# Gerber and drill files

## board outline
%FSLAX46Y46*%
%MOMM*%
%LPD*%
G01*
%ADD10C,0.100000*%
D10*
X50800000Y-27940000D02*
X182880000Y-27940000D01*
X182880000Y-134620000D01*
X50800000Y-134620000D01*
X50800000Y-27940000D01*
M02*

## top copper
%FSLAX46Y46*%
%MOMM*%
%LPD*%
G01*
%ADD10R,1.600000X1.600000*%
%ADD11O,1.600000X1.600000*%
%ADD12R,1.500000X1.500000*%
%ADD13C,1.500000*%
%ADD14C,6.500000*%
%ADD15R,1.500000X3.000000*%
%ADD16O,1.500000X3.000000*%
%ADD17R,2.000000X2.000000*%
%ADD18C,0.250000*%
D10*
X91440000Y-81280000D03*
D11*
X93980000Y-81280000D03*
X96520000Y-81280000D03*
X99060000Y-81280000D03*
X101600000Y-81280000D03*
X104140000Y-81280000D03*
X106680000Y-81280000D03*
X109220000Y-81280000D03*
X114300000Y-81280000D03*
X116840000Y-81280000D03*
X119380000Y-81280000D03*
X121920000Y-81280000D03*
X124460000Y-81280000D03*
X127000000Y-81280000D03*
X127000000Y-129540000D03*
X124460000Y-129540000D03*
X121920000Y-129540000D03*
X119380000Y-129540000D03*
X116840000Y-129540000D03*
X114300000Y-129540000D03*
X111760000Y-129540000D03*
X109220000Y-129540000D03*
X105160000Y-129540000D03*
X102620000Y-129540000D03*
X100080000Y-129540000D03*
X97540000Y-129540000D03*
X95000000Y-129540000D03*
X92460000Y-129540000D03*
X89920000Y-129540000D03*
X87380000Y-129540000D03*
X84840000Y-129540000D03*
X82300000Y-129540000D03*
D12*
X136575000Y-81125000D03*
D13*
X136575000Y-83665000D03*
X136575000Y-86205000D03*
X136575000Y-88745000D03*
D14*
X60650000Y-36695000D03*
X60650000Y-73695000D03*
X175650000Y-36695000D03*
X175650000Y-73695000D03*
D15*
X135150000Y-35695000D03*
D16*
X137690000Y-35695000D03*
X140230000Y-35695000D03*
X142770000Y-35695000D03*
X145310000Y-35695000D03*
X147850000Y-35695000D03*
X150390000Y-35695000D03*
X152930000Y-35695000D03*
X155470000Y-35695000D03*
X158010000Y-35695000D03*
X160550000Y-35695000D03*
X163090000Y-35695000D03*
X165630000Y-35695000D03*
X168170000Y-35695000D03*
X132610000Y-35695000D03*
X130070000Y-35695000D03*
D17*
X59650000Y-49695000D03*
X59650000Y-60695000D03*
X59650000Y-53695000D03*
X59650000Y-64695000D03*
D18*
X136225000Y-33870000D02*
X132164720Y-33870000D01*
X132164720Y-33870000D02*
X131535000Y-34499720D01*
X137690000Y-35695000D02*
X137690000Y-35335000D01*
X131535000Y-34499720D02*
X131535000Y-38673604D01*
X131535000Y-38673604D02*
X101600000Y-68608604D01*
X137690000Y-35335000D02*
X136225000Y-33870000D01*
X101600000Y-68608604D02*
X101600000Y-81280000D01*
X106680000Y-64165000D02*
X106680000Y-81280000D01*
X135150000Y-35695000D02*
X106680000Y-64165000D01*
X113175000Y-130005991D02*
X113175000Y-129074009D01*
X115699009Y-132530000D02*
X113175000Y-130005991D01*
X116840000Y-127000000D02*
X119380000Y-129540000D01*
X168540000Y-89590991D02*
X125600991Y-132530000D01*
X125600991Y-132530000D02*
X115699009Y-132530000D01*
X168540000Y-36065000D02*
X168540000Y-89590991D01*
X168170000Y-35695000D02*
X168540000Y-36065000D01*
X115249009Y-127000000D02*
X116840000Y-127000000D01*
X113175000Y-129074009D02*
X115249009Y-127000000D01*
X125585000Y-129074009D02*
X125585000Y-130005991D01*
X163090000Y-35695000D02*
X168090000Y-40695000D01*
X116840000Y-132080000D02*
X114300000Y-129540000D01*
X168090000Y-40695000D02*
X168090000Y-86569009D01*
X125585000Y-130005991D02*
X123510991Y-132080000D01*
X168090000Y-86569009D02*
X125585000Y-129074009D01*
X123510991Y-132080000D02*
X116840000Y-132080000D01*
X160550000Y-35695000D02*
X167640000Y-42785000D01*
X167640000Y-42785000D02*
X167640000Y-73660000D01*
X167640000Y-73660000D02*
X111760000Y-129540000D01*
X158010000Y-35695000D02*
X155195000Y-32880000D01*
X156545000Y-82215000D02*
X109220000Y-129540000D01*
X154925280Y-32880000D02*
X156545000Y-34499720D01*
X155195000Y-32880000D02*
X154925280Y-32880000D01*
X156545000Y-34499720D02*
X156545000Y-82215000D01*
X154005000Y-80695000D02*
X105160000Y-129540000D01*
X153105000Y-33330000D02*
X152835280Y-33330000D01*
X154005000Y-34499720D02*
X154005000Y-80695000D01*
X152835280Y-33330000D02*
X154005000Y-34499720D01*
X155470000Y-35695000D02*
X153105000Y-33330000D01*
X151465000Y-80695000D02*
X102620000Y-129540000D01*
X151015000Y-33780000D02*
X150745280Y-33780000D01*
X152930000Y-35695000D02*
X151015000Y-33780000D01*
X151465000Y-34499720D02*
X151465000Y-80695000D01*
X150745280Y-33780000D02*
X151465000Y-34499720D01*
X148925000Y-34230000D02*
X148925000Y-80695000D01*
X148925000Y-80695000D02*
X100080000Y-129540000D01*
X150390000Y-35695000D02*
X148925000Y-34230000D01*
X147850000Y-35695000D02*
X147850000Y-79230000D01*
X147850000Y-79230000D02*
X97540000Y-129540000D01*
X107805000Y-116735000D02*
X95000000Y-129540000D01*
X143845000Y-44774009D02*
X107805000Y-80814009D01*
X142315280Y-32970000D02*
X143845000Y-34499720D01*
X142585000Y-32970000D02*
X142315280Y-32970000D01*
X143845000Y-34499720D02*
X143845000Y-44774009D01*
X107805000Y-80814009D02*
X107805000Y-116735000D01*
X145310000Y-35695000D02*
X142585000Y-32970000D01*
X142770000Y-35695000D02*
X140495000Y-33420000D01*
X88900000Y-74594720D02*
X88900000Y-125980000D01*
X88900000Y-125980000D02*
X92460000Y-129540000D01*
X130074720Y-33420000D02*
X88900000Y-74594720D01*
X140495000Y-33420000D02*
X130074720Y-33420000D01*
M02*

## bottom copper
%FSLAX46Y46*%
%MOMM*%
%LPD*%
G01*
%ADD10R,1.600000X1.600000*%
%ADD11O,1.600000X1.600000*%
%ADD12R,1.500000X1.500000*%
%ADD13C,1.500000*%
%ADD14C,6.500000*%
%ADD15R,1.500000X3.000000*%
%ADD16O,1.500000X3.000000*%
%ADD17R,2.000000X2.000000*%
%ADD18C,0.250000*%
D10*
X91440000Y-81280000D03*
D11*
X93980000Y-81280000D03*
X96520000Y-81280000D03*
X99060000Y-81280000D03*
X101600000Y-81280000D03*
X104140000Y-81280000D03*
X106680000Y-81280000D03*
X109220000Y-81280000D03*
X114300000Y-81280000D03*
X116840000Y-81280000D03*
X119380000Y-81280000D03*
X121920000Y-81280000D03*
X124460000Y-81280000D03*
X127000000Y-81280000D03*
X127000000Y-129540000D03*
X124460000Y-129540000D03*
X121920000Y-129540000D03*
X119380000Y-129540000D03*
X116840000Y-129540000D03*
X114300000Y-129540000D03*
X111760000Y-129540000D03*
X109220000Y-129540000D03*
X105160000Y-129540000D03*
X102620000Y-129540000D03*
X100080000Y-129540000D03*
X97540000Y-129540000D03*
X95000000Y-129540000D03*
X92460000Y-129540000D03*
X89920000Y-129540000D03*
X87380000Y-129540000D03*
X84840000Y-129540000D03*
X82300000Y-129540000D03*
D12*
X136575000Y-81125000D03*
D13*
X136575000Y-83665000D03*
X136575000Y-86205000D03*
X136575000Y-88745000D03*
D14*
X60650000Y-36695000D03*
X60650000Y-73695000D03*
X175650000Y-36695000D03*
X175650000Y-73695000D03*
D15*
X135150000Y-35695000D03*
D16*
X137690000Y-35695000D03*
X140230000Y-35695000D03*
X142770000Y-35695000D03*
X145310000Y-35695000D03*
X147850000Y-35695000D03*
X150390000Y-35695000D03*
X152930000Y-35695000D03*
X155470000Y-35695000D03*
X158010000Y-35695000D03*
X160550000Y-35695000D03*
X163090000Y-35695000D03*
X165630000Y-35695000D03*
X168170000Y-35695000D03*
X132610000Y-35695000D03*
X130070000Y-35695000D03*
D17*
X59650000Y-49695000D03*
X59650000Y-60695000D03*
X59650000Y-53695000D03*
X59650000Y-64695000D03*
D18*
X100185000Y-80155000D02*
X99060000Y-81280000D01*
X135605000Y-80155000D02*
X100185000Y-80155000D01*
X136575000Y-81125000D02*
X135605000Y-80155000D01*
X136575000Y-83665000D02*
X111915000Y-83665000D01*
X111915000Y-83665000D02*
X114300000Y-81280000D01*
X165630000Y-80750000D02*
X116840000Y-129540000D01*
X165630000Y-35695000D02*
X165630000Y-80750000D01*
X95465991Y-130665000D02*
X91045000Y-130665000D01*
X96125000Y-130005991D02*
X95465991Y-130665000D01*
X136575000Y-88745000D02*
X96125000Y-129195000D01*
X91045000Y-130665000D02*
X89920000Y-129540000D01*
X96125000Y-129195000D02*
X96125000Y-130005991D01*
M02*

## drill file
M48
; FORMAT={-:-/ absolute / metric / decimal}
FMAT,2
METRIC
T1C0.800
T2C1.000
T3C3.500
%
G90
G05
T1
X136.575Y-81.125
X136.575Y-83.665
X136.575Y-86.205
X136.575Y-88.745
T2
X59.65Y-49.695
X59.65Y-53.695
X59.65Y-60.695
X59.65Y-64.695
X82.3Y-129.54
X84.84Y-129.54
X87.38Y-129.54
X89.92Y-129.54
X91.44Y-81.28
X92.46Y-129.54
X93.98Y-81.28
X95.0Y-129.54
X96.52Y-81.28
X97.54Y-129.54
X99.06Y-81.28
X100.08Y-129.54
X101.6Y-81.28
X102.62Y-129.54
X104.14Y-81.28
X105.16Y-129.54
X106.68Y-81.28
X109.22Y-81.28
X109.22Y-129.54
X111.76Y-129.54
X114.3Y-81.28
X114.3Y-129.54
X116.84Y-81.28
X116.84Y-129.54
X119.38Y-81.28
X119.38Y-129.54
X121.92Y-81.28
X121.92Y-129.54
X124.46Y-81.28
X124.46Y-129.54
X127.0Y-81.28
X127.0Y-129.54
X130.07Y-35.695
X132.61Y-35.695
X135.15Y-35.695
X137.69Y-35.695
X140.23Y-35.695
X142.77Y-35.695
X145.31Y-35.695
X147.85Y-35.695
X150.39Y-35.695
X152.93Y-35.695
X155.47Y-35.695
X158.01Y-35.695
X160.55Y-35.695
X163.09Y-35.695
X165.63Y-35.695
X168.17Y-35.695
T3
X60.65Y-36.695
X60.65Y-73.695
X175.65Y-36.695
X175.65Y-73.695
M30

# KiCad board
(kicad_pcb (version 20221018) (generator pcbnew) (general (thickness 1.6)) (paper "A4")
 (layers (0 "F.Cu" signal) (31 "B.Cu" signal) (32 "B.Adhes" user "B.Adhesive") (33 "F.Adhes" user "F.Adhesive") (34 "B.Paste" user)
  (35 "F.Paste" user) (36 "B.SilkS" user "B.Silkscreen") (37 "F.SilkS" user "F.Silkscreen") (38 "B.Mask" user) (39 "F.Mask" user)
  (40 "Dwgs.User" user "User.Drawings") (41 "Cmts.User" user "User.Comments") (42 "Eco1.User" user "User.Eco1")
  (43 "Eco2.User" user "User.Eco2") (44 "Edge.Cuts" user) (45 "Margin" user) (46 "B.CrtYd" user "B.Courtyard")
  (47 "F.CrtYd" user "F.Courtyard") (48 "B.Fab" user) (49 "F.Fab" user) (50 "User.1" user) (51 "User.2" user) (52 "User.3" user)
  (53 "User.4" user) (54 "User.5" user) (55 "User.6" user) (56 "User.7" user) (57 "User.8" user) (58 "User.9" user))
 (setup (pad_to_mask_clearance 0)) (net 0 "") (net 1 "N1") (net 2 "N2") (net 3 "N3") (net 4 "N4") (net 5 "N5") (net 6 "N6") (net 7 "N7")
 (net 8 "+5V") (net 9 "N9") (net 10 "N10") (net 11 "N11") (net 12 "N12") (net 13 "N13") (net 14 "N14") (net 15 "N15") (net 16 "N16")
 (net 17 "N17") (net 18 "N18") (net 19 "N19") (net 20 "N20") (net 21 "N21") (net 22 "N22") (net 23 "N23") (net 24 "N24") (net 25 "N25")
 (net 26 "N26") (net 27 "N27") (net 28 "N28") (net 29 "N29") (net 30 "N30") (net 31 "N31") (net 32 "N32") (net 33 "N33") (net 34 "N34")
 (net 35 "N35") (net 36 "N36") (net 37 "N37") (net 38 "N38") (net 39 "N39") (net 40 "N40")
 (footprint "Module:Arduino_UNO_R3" (layer "F.Cu") (at 91.44 81.28)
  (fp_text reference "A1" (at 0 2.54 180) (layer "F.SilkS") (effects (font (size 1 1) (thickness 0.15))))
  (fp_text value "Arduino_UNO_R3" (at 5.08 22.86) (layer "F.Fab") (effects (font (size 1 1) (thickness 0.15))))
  (pad "1" thru_hole rect (at 0 0 90) (size 1.6 1.6) (drill 1) (layers "*.Cu" "*.Mask") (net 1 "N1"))
  (pad "2" thru_hole oval (at 2.54 0 90) (size 1.6 1.6) (drill 1) (layers "*.Cu" "*.Mask") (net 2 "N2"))
  (pad "3" thru_hole oval (at 5.08 0 90) (size 1.6 1.6) (drill 1) (layers "*.Cu" "*.Mask") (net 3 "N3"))
  (pad "4" thru_hole oval (at 7.62 0 90) (size 1.6 1.6) (drill 1) (layers "*.Cu" "*.Mask") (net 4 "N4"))
  (pad "5" thru_hole oval (at 10.16 0 90) (size 1.6 1.6) (drill 1) (layers "*.Cu" "*.Mask") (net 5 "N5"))
  (pad "6" thru_hole oval (at 12.7 0 90) (size 1.6 1.6) (drill 1) (layers "*.Cu" "*.Mask") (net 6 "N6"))
  (pad "7" thru_hole oval (at 15.24 0 90) (size 1.6 1.6) (drill 1) (layers "*.Cu" "*.Mask") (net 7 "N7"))
  (pad "8" thru_hole oval (at 17.78 0 90) (size 1.6 1.6) (drill 1) (layers "*.Cu" "*.Mask") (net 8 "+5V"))
  (pad "9" thru_hole oval (at 22.86 0 90) (size 1.6 1.6) (drill 1) (layers "*.Cu" "*.Mask") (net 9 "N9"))
  (pad "10" thru_hole oval (at 25.4 0 90) (size 1.6 1.6) (drill 1) (layers "*.Cu" "*.Mask") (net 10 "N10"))
  (pad "11" thru_hole oval (at 27.94 0 90) (size 1.6 1.6) (drill 1) (layers "*.Cu" "*.Mask") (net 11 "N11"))
  (pad "12" thru_hole oval (at 30.48 0 90) (size 1.6 1.6) (drill 1) (layers "*.Cu" "*.Mask") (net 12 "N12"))
  (pad "13" thru_hole oval (at 33.02 0 90) (size 1.6 1.6) (drill 1) (layers "*.Cu" "*.Mask") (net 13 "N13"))
  (pad "14" thru_hole oval (at 35.56 0 90) (size 1.6 1.6) (drill 1) (layers "*.Cu" "*.Mask") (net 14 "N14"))
  (pad "15" thru_hole oval (at 35.56 48.26 90) (size 1.6 1.6) (drill 1) (layers "*.Cu" "*.Mask") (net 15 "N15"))
  (pad "16" thru_hole oval (at 33.02 48.26 90) (size 1.6 1.6) (drill 1) (layers "*.Cu" "*.Mask") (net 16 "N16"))
  (pad "17" thru_hole oval (at 30.48 48.26 90) (size 1.6 1.6) (drill 1) (layers "*.Cu" "*.Mask") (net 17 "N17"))
  (pad "18" thru_hole oval (at 27.94 48.26 90) (size 1.6 1.6) (drill 1) (layers "*.Cu" "*.Mask") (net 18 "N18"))
  (pad "19" thru_hole oval (at 25.4 48.26 90) (size 1.6 1.6) (drill 1) (layers "*.Cu" "*.Mask") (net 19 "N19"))
  (pad "20" thru_hole oval (at 22.86 48.26 90) (size 1.6 1.6) (drill 1) (layers "*.Cu" "*.Mask") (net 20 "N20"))
  (pad "21" thru_hole oval (at 20.32 48.26 90) (size 1.6 1.6) (drill 1) (layers "*.Cu" "*.Mask") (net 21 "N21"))
  (pad "22" thru_hole oval (at 17.78 48.26 90) (size 1.6 1.6) (drill 1) (layers "*.Cu" "*.Mask") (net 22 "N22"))
  (pad "23" thru_hole oval (at 13.72 48.26 90) (size 1.6 1.6) (drill 1) (layers "*.Cu" "*.Mask") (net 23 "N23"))
  (pad "24" thru_hole oval (at 11.18 48.26 90) (size 1.6 1.6) (drill 1) (layers "*.Cu" "*.Mask") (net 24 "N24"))
  (pad "25" thru_hole oval (at 8.64 48.26 90) (size 1.6 1.6) (drill 1) (layers "*.Cu" "*.Mask") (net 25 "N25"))
  (pad "26" thru_hole oval (at 6.1 48.26 90) (size 1.6 1.6) (drill 1) (layers "*.Cu" "*.Mask") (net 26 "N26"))
  (pad "27" thru_hole oval (at 3.56 48.26 90) (size 1.6 1.6) (drill 1) (layers "*.Cu" "*.Mask") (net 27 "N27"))
  (pad "28" thru_hole oval (at 1.02 48.26 90) (size 1.6 1.6) (drill 1) (layers "*.Cu" "*.Mask") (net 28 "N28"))
  (pad "29" thru_hole oval (at -1.52 48.26 90) (size 1.6 1.6) (drill 1) (layers "*.Cu" "*.Mask") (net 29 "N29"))
  (pad "30" thru_hole oval (at -4.06 48.26 90) (size 1.6 1.6) (drill 1) (layers "*.Cu" "*.Mask") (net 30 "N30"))
  (pad "31" thru_hole oval (at -6.6 48.26 90) (size 1.6 1.6) (drill 1) (layers "*.Cu" "*.Mask") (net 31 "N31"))
  (pad "32" thru_hole oval (at -9.14 48.26 90) (size 1.6 1.6) (drill 1) (layers "*.Cu" "*.Mask") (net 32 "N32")))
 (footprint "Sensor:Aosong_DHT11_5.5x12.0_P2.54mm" (layer "F.Cu") (at 136.575 81.125)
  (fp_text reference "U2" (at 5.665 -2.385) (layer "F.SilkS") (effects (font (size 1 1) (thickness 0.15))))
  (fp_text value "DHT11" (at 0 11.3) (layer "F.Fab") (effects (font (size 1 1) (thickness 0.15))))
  (pad "1" thru_hole rect (at 0 0) (size 1.5 1.5) (drill 0.8) (layers "*.Cu" "*.Mask") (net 4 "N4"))
  (pad "2" thru_hole circle (at 0 2.54) (size 1.5 1.5) (drill 0.8) (layers "*.Cu" "*.Mask") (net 9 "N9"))
  (pad "3" thru_hole circle (at 0 5.08) (size 1.5 1.5) (drill 0.8) (layers "*.Cu" "*.Mask") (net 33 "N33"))
  (pad "4" thru_hole circle (at 0 7.62) (size 1.5 1.5) (drill 0.8) (layers "*.Cu" "*.Mask") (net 29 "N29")))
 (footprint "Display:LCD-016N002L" (layer "F.Cu") (at 135.15 35.695)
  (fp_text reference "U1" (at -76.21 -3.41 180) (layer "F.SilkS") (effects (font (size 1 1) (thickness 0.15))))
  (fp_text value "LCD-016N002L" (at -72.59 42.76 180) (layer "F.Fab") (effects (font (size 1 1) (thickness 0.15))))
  (pad "" thru_hole circle (at -74.5 1 180) (size 6.5 6.5) (drill 3.5) (layers "*.Cu" "*.Mask"))
  (pad "" thru_hole circle (at -74.5 38 180) (size 6.5 6.5) (drill 3.5) (layers "*.Cu" "*.Mask"))
  (pad "" thru_hole circle (at 40.5 1 180) (size 6.5 6.5) (drill 3.5) (layers "*.Cu" "*.Mask"))
  (pad "" thru_hole circle (at 40.5 38 180) (size 6.5 6.5) (drill 3.5) (layers "*.Cu" "*.Mask"))
  (pad "1" thru_hole rect (at 0 0 180) (size 1.5 3) (drill 1) (layers "*.Cu" "*.Mask") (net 7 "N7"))
  (pad "2" thru_hole oval (at 2.54 0 180) (size 1.5 3) (drill 1) (layers "*.Cu" "*.Mask") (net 5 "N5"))
  (pad "3" thru_hole oval (at 5.08 0 180) (size 1.5 3) (drill 1) (layers "*.Cu" "*.Mask") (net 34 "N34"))
  (pad "4" thru_hole oval (at 7.62 0 180) (size 1.5 3) (drill 1) (layers "*.Cu" "*.Mask") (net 28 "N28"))
  (pad "5" thru_hole oval (at 10.16 0 180) (size 1.5 3) (drill 1) (layers "*.Cu" "*.Mask") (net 27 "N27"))
  (pad "6" thru_hole oval (at 12.7 0 180) (size 1.5 3) (drill 1) (layers "*.Cu" "*.Mask") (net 26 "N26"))
  (pad "7" thru_hole oval (at 15.24 0 180) (size 1.5 3) (drill 1) (layers "*.Cu" "*.Mask") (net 25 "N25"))
  (pad "8" thru_hole oval (at 17.78 0 180) (size 1.5 3) (drill 1) (layers "*.Cu" "*.Mask") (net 24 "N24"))
  (pad "9" thru_hole oval (at 20.32 0 180) (size 1.5 3) (drill 1) (layers "*.Cu" "*.Mask") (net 23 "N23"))
  (pad "10" thru_hole oval (at 22.86 0 180) (size 1.5 3) (drill 1) (layers "*.Cu" "*.Mask") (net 22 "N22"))
  (pad "11" thru_hole oval (at 25.4 0 180) (size 1.5 3) (drill 1) (layers "*.Cu" "*.Mask") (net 21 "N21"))
  (pad "12" thru_hole oval (at 27.94 0 180) (size 1.5 3) (drill 1) (layers "*.Cu" "*.Mask") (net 20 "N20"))
  (pad "13" thru_hole oval (at 30.48 0 180) (size 1.5 3) (drill 1) (layers "*.Cu" "*.Mask") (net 19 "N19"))
  (pad "14" thru_hole oval (at 33.02 0 180) (size 1.5 3) (drill 1) (layers "*.Cu" "*.Mask") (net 18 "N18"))
  (pad "15" thru_hole oval (at -2.54 0 180) (size 1.5 3) (drill 1) (layers "*.Cu" "*.Mask") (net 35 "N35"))
  (pad "16" thru_hole oval (at -5.08 0 180) (size 1.5 3) (drill 1) (layers "*.Cu" "*.Mask") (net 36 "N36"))
  (pad "A1" thru_hole rect (at -75.5 14 180) (size 2 2) (drill 1) (layers "*.Cu" "*.Mask") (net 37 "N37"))
  (pad "A2" thru_hole rect (at -75.5 25 180) (size 2 2) (drill 1) (layers "*.Cu" "*.Mask") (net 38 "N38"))
  (pad "K1" thru_hole rect (at -75.5 18 180) (size 2 2) (drill 1) (layers "*.Cu" "*.Mask") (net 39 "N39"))
  (pad "K2" thru_hole rect (at -75.5 29 180) (size 2 2) (drill 1) (layers "*.Cu" "*.Mask") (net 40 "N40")))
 (gr_rect (start 50.8 27.94) (end 182.88 134.62) (stroke (width 0.1) (type default)) (fill none) (layer "Edge.Cuts"))
 (segment (start 100.185 80.155) (end 99.06 81.28) (width 0.25) (layer "B.Cu") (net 4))
 (segment (start 135.605 80.155) (end 100.185 80.155) (width 0.25) (layer "B.Cu") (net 4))
 (segment (start 136.575 81.125) (end 135.605 80.155) (width 0.25) (layer "B.Cu") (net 4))
 (segment (start 136.225 33.87) (end 132.16472 33.87) (width 0.25) (layer "F.Cu") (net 5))
 (segment (start 132.16472 33.87) (end 131.535 34.49972) (width 0.25) (layer "F.Cu") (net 5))
 (segment (start 137.69 35.695) (end 137.69 35.335) (width 0.25) (layer "F.Cu") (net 5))
 (segment (start 131.535 34.49972) (end 131.535 38.673604) (width 0.25) (layer "F.Cu") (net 5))
 (segment (start 131.535 38.673604) (end 101.6 68.608604) (width 0.25) (layer "F.Cu") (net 5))
 (segment (start 137.69 35.335) (end 136.225 33.87) (width 0.25) (layer "F.Cu") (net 5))
 (segment (start 101.6 68.608604) (end 101.6 81.28) (width 0.25) (layer "F.Cu") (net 5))
 (segment (start 106.68 64.165) (end 106.68 81.28) (width 0.25) (layer "F.Cu") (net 7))
 (segment (start 135.15 35.695) (end 106.68 64.165) (width 0.25) (layer "F.Cu") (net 7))
 (segment (start 136.575 83.665) (end 111.915 83.665) (width 0.25) (layer "B.Cu") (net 9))
 (segment (start 111.915 83.665) (end 114.3 81.28) (width 0.25) (layer "B.Cu") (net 9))
 (segment (start 113.175 130.005991) (end 113.175 129.074009) (width 0.25) (layer "F.Cu") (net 18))
 (segment (start 115.699009 132.53) (end 113.175 130.005991) (width 0.25) (layer "F.Cu") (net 18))
 (segment (start 116.84 127) (end 119.38 129.54) (width 0.25) (layer "F.Cu") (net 18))
 (segment (start 168.54 89.590991) (end 125.600991 132.53) (width 0.25) (layer "F.Cu") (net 18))
 (segment (start 125.600991 132.53) (end 115.699009 132.53) (width 0.25) (layer "F.Cu") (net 18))
 (segment (start 168.54 36.065) (end 168.54 89.590991) (width 0.25) (layer "F.Cu") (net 18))
 (segment (start 168.17 35.695) (end 168.54 36.065) (width 0.25) (layer "F.Cu") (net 18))
 (segment (start 115.249009 127) (end 116.84 127) (width 0.25) (layer "F.Cu") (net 18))
 (segment (start 113.175 129.074009) (end 115.249009 127) (width 0.25) (layer "F.Cu") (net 18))
 (segment (start 165.63 80.75) (end 116.84 129.54) (width 0.25) (layer "B.Cu") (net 19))
 (segment (start 165.63 35.695) (end 165.63 80.75) (width 0.25) (layer "B.Cu") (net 19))
 (segment (start 125.585 129.074009) (end 125.585 130.005991) (width 0.25) (layer "F.Cu") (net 20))
 (segment (start 163.09 35.695) (end 168.09 40.695) (width 0.25) (layer "F.Cu") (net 20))
 (segment (start 116.84 132.08) (end 114.3 129.54) (width 0.25) (layer "F.Cu") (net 20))
 (segment (start 168.09 40.695) (end 168.09 86.569009) (width 0.25) (layer "F.Cu") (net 20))
 (segment (start 125.585 130.005991) (end 123.510991 132.08) (width 0.25) (layer "F.Cu") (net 20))
 (segment (start 168.09 86.569009) (end 125.585 129.074009) (width 0.25) (layer "F.Cu") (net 20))
 (segment (start 123.510991 132.08) (end 116.84 132.08) (width 0.25) (layer "F.Cu") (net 20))
 (segment (start 160.55 35.695) (end 167.64 42.785) (width 0.25) (layer "F.Cu") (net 21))
 (segment (start 167.64 42.785) (end 167.64 73.66) (width 0.25) (layer "F.Cu") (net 21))
 (segment (start 167.64 73.66) (end 111.76 129.54) (width 0.25) (layer "F.Cu") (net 21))
 (segment (start 158.01 35.695) (end 155.195 32.88) (width 0.25) (layer "F.Cu") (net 22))
 (segment (start 156.545 82.215) (end 109.22 129.54) (width 0.25) (layer "F.Cu") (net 22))
 (segment (start 154.92528 32.88) (end 156.545 34.49972) (width 0.25) (layer "F.Cu") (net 22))
 (segment (start 155.195 32.88) (end 154.92528 32.88) (width 0.25) (layer "F.Cu") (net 22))
 (segment (start 156.545 34.49972) (end 156.545 82.215) (width 0.25) (layer "F.Cu") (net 22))
 (segment (start 154.005 80.695) (end 105.16 129.54) (width 0.25) (layer "F.Cu") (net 23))
 (segment (start 153.105 33.33) (end 152.83528 33.33) (width 0.25) (layer "F.Cu") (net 23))
 (segment (start 154.005 34.49972) (end 154.005 80.695) (width 0.25) (layer "F.Cu") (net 23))
 (segment (start 152.83528 33.33) (end 154.005 34.49972) (width 0.25) (layer "F.Cu") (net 23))
 (segment (start 155.47 35.695) (end 153.105 33.33) (width 0.25) (layer "F.Cu") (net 23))
 (segment (start 151.465 80.695) (end 102.62 129.54) (width 0.25) (layer "F.Cu") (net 24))
 (segment (start 151.015 33.78) (end 150.74528 33.78) (width 0.25) (layer "F.Cu") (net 24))
 (segment (start 152.93 35.695) (end 151.015 33.78) (width 0.25) (layer "F.Cu") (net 24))
 (segment (start 151.465 34.49972) (end 151.465 80.695) (width 0.25) (layer "F.Cu") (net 24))
 (segment (start 150.74528 33.78) (end 151.465 34.49972) (width 0.25) (layer "F.Cu") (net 24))
 (segment (start 148.925 34.23) (end 148.925 80.695) (width 0.25) (layer "F.Cu") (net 25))
 (segment (start 148.925 80.695) (end 100.08 129.54) (width 0.25) (layer "F.Cu") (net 25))
 (segment (start 150.39 35.695) (end 148.925 34.23) (width 0.25) (layer "F.Cu") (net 25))
 (segment (start 147.85 35.695) (end 147.85 79.23) (width 0.25) (layer "F.Cu") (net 26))
 (segment (start 147.85 79.23) (end 97.54 129.54) (width 0.25) (layer "F.Cu") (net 26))
 (segment (start 107.805 116.735) (end 95 129.54) (width 0.25) (layer "F.Cu") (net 27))
 (segment (start 143.845 44.774009) (end 107.805 80.814009) (width 0.25) (layer "F.Cu") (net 27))
 (segment (start 142.31528 32.97) (end 143.845 34.49972) (width 0.25) (layer "F.Cu") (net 27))
 (segment (start 142.585 32.97) (end 142.31528 32.97) (width 0.25) (layer "F.Cu") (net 27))
 (segment (start 143.845 34.49972) (end 143.845 44.774009) (width 0.25) (layer "F.Cu") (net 27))
 (segment (start 107.805 80.814009) (end 107.805 116.735) (width 0.25) (layer "F.Cu") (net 27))
 (segment (start 145.31 35.695) (end 142.585 32.97) (width 0.25) (layer "F.Cu") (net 27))
 (segment (start 142.77 35.695) (end 140.495 33.42) (width 0.25) (layer "F.Cu") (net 28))
 (segment (start 88.9 74.59472) (end 88.9 125.98) (width 0.25) (layer "F.Cu") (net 28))
 (segment (start 88.9 125.98) (end 92.46 129.54) (width 0.25) (layer "F.Cu") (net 28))
 (segment (start 130.07472 33.42) (end 88.9 74.59472) (width 0.25) (layer "F.Cu") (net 28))
 (segment (start 140.495 33.42) (end 130.07472 33.42) (width 0.25) (layer "F.Cu") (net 28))
 (segment (start 95.465991 130.665) (end 91.045 130.665) (width 0.25) (layer "B.Cu") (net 29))
 (segment (start 96.125 130.005991) (end 95.465991 130.665) (width 0.25) (layer "B.Cu") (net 29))
 (segment (start 136.575 88.745) (end 96.125 129.195) (width 0.25) (layer "B.Cu") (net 29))
 (segment (start 91.045 130.665) (end 89.92 129.54) (width 0.25) (layer "B.Cu") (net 29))
 (segment (start 96.125 129.195) (end 96.125 130.005991) (width 0.25) (layer "B.Cu") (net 29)))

